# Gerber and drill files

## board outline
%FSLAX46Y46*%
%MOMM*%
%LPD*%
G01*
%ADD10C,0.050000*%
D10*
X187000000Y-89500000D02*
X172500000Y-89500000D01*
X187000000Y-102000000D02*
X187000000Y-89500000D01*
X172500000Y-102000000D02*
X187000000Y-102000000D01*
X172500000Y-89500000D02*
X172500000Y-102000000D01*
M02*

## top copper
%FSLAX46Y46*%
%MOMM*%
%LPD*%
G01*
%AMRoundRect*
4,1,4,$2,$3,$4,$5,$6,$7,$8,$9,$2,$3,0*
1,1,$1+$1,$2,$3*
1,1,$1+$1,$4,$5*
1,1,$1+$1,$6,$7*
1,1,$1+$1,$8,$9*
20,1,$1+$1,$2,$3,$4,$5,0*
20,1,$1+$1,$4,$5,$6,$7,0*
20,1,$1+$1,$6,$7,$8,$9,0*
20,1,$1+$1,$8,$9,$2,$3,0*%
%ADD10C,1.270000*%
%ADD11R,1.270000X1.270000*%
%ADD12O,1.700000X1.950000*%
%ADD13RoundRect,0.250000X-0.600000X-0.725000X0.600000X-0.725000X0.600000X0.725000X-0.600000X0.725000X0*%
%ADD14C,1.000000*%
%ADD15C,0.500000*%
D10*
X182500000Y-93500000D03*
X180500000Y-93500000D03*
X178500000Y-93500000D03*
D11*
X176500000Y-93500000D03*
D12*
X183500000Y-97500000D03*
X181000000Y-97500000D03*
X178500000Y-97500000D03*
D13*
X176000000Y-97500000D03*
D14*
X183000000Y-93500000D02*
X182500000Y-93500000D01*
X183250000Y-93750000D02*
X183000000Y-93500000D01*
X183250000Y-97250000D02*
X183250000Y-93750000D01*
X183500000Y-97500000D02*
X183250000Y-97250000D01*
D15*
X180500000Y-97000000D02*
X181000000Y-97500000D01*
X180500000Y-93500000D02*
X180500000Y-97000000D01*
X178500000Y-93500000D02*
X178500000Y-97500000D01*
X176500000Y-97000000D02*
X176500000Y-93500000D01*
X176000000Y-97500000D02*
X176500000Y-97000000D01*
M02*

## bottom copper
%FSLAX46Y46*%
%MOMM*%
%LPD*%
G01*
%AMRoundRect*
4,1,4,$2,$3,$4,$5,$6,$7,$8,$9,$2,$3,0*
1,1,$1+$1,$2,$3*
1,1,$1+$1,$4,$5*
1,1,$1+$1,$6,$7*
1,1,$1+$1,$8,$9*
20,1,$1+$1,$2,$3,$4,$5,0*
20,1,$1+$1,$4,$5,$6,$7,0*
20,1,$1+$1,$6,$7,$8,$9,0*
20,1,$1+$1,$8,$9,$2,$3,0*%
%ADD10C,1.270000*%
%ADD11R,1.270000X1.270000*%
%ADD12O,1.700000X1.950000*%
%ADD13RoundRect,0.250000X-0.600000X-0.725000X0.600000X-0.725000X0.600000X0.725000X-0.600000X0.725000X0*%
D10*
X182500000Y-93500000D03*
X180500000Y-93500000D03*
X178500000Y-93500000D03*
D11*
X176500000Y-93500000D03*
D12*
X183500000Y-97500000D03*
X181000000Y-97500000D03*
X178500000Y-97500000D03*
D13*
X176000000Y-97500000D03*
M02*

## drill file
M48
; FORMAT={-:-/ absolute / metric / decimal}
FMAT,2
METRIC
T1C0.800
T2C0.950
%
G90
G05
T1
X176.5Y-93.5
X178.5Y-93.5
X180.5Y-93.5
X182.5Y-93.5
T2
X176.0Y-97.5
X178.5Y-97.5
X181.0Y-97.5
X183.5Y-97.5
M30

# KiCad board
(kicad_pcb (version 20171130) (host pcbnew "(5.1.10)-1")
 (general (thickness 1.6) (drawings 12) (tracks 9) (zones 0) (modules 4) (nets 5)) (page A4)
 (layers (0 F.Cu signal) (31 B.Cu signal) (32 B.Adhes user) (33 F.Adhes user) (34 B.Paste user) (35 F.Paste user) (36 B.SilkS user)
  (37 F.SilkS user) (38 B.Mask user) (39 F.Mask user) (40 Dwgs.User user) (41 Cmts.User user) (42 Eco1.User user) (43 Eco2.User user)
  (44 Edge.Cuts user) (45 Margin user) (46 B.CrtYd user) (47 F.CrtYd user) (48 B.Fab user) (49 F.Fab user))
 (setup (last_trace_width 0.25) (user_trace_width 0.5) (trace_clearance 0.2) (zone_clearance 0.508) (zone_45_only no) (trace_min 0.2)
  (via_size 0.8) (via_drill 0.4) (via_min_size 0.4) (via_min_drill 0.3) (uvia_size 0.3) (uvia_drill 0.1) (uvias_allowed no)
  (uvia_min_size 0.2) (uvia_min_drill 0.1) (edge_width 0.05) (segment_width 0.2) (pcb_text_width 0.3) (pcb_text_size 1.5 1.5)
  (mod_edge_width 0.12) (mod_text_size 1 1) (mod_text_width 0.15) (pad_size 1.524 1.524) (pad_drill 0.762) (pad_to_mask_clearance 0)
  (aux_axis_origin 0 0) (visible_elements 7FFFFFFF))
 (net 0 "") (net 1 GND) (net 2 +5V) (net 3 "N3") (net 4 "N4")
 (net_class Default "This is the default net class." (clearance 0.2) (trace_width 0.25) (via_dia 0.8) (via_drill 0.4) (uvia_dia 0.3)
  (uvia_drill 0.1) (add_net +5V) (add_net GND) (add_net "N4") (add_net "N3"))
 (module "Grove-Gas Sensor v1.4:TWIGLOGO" (layer B.Cu) (at 184.5 94)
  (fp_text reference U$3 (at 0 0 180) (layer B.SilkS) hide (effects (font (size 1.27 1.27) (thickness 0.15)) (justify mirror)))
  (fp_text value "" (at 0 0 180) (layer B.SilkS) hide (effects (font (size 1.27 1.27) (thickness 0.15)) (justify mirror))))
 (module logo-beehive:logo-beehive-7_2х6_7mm (layer F.Cu) (at 176 93.5 270)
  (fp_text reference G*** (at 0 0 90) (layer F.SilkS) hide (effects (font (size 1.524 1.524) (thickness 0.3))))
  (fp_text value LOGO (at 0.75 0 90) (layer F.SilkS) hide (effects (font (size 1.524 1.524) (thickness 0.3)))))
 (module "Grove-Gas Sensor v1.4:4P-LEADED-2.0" (layer B.Cu) (at 179.5 93.5)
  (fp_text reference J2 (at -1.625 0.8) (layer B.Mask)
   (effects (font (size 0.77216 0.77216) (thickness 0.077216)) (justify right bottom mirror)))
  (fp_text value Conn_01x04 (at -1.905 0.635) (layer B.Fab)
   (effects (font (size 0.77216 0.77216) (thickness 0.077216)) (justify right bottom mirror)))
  (pad 4 thru_hole circle (at 3 0) (size 1.27 1.27) (drill 0.8) (layers *.Cu *.Mask) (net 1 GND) (solder_mask_margin 0.0508))
  (pad 3 thru_hole circle (at 1 0) (size 1.27 1.27) (drill 0.8) (layers *.Cu *.Mask) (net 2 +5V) (solder_mask_margin 0.0508))
  (pad 2 thru_hole circle (at -1 0) (size 1.27 1.27) (drill 0.8) (layers *.Cu *.Mask) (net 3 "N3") (solder_mask_margin 0.0508))
  (pad 1 thru_hole rect (at -3 0) (size 1.27 1.27) (drill 0.8) (layers *.Cu *.Mask) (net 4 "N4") (solder_mask_margin 0.0508)))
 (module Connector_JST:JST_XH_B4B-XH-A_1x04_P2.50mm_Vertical (layer F.Cu) (at 176 97.5)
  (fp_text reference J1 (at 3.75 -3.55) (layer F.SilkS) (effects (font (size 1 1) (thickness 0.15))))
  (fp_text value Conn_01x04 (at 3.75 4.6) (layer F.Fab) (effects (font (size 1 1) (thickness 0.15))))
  (pad 4 thru_hole oval (at 7.5 0) (size 1.7 1.95) (drill 0.95) (layers *.Cu *.Mask) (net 1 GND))
  (pad 3 thru_hole oval (at 5 0) (size 1.7 1.95) (drill 0.95) (layers *.Cu *.Mask) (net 2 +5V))
  (pad 2 thru_hole oval (at 2.5 0) (size 1.7 1.95) (drill 0.95) (layers *.Cu *.Mask) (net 3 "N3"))
  (pad 1 thru_hole roundrect (at 0 0) (size 1.7 1.95) (drill 0.95) (layers *.Cu *.Mask) (roundrect_rratio 0.1470588235294118) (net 4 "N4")))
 (gr_line (start 187 89.5) (end 172.5 89.5) (layer Edge.Cuts) (width 0.05))
 (gr_line (start 187 102) (end 187 89.5) (layer Edge.Cuts) (width 0.05))
 (gr_line (start 172.5 102) (end 187 102) (layer Edge.Cuts) (width 0.05))
 (gr_line (start 172.5 89.5) (end 172.5 102) (layer Edge.Cuts) (width 0.05))
 (segment (start 183 93.5) (end 182.5 93.5) (width 1) (layer F.Cu) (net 1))
 (segment (start 183.25 93.75) (end 183 93.5) (width 1) (layer F.Cu) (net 1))
 (segment (start 183.25 97.25) (end 183.25 93.75) (width 1) (layer F.Cu) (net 1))
 (segment (start 183.5 97.5) (end 183.25 97.25) (width 1) (layer F.Cu) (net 1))
 (segment (start 180.5 97) (end 181 97.5) (width 0.5) (layer F.Cu) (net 2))
 (segment (start 180.5 93.5) (end 180.5 97) (width 0.5) (layer F.Cu) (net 2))
 (segment (start 178.5 93.5) (end 178.5 97.5) (width 0.5) (layer F.Cu) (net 3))
 (segment (start 176.5 97) (end 176.5 93.5) (width 0.5) (layer F.Cu) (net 4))
 (segment (start 176 97.5) (end 176.5 97) (width 0.5) (layer F.Cu) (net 4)))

